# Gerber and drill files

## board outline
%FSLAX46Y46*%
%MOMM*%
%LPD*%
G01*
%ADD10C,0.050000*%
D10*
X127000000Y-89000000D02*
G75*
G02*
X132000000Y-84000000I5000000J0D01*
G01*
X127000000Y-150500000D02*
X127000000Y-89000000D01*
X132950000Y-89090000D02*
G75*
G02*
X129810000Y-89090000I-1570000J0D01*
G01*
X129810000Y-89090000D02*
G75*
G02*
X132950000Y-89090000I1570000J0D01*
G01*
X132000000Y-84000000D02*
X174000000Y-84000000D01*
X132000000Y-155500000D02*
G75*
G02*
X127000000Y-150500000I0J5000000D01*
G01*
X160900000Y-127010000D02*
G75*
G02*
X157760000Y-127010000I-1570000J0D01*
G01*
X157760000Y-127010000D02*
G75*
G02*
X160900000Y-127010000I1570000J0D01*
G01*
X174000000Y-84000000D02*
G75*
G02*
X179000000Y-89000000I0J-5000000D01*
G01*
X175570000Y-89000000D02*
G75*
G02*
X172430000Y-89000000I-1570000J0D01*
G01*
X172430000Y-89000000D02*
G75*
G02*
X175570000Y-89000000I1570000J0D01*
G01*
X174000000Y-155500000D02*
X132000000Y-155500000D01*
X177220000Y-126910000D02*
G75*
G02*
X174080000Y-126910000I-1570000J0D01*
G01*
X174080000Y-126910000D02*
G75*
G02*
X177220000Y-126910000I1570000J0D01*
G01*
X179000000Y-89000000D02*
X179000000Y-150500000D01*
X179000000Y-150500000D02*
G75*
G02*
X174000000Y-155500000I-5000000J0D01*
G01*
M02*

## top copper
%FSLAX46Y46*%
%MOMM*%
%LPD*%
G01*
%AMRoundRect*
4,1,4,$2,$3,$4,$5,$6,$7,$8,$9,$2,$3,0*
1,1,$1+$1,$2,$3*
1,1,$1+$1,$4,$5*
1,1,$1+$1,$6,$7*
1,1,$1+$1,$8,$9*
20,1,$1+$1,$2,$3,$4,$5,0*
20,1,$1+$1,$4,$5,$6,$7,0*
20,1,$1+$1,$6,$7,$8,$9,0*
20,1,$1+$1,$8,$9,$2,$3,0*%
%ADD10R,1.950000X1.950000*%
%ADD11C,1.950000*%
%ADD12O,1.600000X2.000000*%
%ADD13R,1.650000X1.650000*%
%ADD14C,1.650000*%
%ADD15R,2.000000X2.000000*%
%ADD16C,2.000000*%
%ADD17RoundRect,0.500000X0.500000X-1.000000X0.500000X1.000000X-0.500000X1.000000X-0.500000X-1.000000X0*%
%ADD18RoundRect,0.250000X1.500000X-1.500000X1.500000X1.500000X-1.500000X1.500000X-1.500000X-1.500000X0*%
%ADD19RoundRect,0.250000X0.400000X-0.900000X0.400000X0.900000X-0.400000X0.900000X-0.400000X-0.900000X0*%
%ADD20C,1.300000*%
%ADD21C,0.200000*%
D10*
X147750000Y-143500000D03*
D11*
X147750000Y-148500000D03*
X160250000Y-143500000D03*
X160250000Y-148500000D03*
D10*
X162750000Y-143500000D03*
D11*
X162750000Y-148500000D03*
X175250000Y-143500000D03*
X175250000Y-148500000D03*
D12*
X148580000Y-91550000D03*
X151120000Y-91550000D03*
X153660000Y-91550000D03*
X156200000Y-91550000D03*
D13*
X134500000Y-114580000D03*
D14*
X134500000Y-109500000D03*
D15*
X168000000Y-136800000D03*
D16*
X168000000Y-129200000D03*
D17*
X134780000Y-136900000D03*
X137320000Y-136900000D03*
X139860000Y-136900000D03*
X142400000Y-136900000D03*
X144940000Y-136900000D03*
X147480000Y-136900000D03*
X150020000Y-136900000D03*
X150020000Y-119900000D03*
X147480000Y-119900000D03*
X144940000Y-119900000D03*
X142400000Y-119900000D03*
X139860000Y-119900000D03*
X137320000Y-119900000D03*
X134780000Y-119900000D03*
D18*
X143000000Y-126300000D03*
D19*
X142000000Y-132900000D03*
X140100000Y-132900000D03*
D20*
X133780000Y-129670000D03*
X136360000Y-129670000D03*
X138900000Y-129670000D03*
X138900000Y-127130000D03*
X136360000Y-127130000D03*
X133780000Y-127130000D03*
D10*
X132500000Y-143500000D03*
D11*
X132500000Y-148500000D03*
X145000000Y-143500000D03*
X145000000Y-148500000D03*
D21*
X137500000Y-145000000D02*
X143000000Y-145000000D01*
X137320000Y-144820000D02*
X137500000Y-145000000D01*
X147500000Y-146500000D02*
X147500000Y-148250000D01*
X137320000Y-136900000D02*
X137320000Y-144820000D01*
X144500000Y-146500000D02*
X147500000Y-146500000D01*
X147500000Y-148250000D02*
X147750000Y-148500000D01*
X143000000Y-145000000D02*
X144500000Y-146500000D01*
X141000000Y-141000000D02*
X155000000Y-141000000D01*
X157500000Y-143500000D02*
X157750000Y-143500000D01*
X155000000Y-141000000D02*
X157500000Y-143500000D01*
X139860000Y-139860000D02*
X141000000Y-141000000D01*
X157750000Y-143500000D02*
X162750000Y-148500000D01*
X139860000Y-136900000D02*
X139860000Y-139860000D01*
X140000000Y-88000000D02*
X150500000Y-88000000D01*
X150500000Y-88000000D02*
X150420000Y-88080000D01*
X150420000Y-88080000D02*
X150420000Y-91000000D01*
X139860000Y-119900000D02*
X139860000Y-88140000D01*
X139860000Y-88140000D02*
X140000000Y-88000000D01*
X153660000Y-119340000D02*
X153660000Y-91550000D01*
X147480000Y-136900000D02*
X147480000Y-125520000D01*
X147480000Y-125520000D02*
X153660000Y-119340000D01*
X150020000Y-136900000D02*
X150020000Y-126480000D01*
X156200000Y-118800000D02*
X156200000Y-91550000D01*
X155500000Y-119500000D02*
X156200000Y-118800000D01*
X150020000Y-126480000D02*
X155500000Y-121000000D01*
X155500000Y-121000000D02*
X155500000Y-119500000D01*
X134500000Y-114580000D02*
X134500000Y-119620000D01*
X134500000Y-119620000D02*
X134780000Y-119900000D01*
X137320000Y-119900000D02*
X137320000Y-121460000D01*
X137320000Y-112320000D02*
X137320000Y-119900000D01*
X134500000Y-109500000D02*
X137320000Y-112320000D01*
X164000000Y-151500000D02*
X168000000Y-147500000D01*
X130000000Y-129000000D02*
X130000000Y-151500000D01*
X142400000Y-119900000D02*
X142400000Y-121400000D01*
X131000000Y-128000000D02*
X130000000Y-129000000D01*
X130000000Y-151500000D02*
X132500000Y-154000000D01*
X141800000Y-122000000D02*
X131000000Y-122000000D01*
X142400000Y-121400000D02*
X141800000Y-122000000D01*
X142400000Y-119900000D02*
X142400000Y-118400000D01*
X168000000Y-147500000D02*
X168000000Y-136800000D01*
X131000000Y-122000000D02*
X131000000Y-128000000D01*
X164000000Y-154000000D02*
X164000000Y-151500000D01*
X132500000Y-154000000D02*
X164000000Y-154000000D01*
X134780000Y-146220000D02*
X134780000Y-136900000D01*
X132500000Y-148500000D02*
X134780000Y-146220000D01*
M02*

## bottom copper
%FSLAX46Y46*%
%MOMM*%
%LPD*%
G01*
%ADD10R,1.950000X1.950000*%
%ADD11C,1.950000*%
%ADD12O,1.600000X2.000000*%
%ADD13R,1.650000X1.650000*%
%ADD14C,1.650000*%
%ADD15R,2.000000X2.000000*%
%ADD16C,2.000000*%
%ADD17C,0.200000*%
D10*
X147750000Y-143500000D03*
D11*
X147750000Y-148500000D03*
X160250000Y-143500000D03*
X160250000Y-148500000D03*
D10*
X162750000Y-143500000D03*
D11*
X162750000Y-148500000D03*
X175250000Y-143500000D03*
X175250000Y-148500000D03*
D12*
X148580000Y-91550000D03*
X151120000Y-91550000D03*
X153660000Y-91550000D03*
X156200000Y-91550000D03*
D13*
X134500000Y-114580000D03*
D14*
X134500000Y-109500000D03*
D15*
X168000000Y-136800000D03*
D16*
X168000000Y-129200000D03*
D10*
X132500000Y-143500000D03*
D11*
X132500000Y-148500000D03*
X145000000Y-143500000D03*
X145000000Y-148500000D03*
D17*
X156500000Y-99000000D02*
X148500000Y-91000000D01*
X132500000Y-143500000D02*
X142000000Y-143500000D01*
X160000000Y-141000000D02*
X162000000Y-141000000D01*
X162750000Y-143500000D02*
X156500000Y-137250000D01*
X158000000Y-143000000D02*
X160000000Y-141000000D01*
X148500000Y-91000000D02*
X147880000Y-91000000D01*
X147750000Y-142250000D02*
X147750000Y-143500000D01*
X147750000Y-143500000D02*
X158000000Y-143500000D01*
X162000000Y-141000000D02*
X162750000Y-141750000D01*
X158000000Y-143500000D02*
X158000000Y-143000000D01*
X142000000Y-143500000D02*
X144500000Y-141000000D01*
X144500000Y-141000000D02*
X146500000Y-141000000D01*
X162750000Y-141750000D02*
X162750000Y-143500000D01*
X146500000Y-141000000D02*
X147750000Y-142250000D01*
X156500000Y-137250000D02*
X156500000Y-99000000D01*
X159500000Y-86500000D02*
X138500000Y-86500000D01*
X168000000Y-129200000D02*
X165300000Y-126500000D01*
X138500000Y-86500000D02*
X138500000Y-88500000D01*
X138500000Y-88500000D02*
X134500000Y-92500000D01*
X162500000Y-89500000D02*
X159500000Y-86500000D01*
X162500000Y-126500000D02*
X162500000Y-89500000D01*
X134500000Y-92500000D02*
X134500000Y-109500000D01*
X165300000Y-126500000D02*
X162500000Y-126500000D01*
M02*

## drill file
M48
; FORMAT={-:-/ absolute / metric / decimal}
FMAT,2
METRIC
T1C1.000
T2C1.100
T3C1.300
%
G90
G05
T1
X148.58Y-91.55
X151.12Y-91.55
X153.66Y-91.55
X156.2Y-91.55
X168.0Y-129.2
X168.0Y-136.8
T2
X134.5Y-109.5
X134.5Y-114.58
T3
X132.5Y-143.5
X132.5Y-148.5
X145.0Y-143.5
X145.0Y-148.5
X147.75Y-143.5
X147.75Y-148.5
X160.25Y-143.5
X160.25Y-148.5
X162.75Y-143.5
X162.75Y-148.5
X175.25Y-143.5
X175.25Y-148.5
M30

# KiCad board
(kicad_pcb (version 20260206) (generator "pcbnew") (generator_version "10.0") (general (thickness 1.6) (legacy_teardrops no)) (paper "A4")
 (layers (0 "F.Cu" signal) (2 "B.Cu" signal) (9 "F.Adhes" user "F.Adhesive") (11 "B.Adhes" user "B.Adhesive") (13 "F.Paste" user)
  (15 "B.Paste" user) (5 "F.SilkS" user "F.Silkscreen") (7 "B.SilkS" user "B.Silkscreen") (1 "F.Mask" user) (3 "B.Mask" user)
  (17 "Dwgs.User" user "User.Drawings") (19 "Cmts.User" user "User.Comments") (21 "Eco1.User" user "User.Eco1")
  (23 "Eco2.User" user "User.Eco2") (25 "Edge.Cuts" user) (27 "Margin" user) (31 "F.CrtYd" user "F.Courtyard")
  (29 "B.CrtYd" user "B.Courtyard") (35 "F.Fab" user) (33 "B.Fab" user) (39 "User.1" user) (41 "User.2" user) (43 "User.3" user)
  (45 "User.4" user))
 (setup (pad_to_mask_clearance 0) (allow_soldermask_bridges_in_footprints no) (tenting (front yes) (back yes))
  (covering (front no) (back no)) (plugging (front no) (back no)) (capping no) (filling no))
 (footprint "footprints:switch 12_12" (layer "F.Cu") (at 154 146)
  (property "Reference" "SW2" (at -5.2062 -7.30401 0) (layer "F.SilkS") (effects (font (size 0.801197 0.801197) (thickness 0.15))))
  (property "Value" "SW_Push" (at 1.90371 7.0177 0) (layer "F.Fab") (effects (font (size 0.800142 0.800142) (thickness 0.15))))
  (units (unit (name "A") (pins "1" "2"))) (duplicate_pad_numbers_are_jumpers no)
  (pad "1" thru_hole rect (at -6.25 -2.5) (size 1.95 1.95) (drill 1.3) (layers "*.Cu" "*.Mask") (remove_unused_layers no) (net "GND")
   (solder_mask_margin 0.102))
  (pad "2" thru_hole circle (at -6.25 2.5) (size 1.95 1.95) (drill 1.3) (layers "*.Cu" "*.Mask") (remove_unused_layers no)
   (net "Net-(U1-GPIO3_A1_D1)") (solder_mask_margin 0.102))
  (pad "3" thru_hole circle (at 6.25 -2.5) (size 1.95 1.95) (drill 1.3) (layers "*.Cu" "*.Mask") (remove_unused_layers no)
   (solder_mask_margin 0.102))
  (pad "4" thru_hole circle (at 6.25 2.5) (size 1.95 1.95) (drill 1.3) (layers "*.Cu" "*.Mask") (remove_unused_layers no)
   (solder_mask_margin 0.102)))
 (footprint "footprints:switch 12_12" (layer "F.Cu") (at 169 146)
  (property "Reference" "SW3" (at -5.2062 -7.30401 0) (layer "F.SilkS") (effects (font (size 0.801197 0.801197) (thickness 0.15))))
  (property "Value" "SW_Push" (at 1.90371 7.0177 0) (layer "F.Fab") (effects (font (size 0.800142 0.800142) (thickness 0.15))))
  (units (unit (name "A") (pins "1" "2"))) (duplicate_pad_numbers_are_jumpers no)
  (pad "1" thru_hole rect (at -6.25 -2.5) (size 1.95 1.95) (drill 1.3) (layers "*.Cu" "*.Mask") (remove_unused_layers no) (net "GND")
   (solder_mask_margin 0.102))
  (pad "2" thru_hole circle (at -6.25 2.5) (size 1.95 1.95) (drill 1.3) (layers "*.Cu" "*.Mask") (remove_unused_layers no)
   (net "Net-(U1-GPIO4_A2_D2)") (solder_mask_margin 0.102))
  (pad "3" thru_hole circle (at 6.25 -2.5) (size 1.95 1.95) (drill 1.3) (layers "*.Cu" "*.Mask") (remove_unused_layers no)
   (solder_mask_margin 0.102))
  (pad "4" thru_hole circle (at 6.25 2.5) (size 1.95 1.95) (drill 1.3) (layers "*.Cu" "*.Mask") (remove_unused_layers no)
   (solder_mask_margin 0.102)))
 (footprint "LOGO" (layer "F.Cu") (at 171 118)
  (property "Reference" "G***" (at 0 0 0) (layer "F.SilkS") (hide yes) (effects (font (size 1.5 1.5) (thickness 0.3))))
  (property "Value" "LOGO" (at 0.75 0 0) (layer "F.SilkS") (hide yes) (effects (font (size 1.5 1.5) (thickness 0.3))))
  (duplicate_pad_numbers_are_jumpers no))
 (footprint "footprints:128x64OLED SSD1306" (layer "F.Cu") (at 152.2 102.15)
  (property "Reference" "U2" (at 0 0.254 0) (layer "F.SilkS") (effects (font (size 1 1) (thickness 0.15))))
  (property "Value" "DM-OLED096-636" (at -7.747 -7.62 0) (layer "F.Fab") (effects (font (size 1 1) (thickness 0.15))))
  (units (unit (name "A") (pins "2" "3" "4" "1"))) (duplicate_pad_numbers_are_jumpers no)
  (pad "1" thru_hole oval (at -3.62 -10.6 90) (size 2 1.6) (drill 1) (layers "*.Cu" "*.Mask") (remove_unused_layers no) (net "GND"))
  (pad "2" thru_hole oval (at -1.08 -10.6 90) (size 2 1.6) (drill 1) (layers "*.Cu" "*.Mask") (remove_unused_layers no) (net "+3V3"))
  (pad "3" thru_hole oval (at 1.46 -10.6 90) (size 2 1.6) (drill 1) (layers "*.Cu" "*.Mask") (remove_unused_layers no)
   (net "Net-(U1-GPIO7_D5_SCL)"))
  (pad "4" thru_hole oval (at 4 -10.6 90) (size 2 1.6) (drill 1) (layers "*.Cu" "*.Mask") (remove_unused_layers no)
   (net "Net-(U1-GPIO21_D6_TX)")))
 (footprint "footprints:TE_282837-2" (layer "F.Cu") (at 134.5 112.04 90)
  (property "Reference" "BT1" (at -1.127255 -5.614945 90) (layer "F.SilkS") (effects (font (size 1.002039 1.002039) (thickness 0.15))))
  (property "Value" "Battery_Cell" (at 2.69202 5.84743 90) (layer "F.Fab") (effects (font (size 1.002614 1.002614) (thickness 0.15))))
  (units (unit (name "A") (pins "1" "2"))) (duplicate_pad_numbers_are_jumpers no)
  (pad "1" thru_hole rect (at -2.54 0 90) (size 1.65 1.65) (drill 1.1) (layers "*.Cu" "*.Mask") (remove_unused_layers no)
   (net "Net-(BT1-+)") (solder_mask_margin 0.102))
  (pad "2" thru_hole circle (at 2.54 0 90) (size 1.65 1.65) (drill 1.1) (layers "*.Cu" "*.Mask") (remove_unused_layers no)
   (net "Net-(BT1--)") (solder_mask_margin 0.102)))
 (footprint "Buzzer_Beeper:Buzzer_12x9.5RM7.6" (layer "F.Cu") (at 168 136.8 90)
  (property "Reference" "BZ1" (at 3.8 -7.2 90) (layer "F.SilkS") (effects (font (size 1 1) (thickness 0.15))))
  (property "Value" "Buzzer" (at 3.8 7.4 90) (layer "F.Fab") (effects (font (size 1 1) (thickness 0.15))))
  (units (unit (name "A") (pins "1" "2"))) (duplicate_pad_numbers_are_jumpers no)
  (pad "1" thru_hole rect (at 0 0 90) (size 2 2) (drill 1) (layers "*.Cu" "*.Mask") (remove_unused_layers no) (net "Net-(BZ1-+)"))
  (pad "2" thru_hole circle (at 7.6 0 90) (size 2 2) (drill 1) (layers "*.Cu" "*.Mask") (remove_unused_layers no) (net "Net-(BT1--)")))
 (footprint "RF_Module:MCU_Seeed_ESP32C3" (layer "F.Cu") (at 142.4 128.4 90)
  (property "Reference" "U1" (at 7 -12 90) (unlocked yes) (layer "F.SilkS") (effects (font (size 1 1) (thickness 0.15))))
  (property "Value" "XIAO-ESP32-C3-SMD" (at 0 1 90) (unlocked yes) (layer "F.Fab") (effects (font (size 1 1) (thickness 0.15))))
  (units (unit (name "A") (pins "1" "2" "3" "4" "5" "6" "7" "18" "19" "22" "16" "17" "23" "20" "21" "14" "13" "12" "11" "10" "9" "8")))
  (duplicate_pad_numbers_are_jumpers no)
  (pad "" smd roundrect (at 1.1 -0.4 90) (size 1.5 1.5) (layers "F.Paste") (roundrect_rratio 0.1666666667))
  (pad "" smd roundrect (at 1.1 1.6 90) (size 1.5 1.5) (layers "F.Paste") (roundrect_rratio 0.1666666667))
  (pad "" smd roundrect (at 3.1 -0.4 90) (size 1.5 1.5) (layers "F.Paste") (roundrect_rratio 0.1666666667))
  (pad "" smd roundrect (at 3.1 1.6 90) (size 1.5 1.5) (layers "F.Paste") (roundrect_rratio 0.1666666667))
  (pad "1" smd roundrect (at -8.5 -7.62 90) (size 3 2) (layers "F.Cu" "F.Mask" "F.Paste") (roundrect_rratio 0.25)
   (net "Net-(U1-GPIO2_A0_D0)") (thermal_bridge_angle 45))
  (pad "2" smd roundrect (at -8.5 -5.08 90) (size 3 2) (layers "F.Cu" "F.Mask" "F.Paste") (roundrect_rratio 0.25)
   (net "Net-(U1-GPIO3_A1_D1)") (thermal_bridge_angle 45))
  (pad "3" smd roundrect (at -8.5 -2.54 90) (size 3 2) (layers "F.Cu" "F.Mask" "F.Paste") (roundrect_rratio 0.25)
   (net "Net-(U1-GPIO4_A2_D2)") (thermal_bridge_angle 45))
  (pad "4" smd roundrect (at -8.5 0 90) (size 3 2) (layers "F.Cu" "F.Mask" "F.Paste") (roundrect_rratio 0.25)
   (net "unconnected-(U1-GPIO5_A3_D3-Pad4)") (thermal_bridge_angle 45))
  (pad "5" smd roundrect (at -8.5 2.54 90) (size 3 2) (layers "F.Cu" "F.Mask" "F.Paste") (roundrect_rratio 0.25)
   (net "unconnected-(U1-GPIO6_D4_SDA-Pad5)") (thermal_bridge_angle 45))
  (pad "6" smd roundrect (at -8.5 5.08 90) (size 3 2) (layers "F.Cu" "F.Mask" "F.Paste") (roundrect_rratio 0.25)
   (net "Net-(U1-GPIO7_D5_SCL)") (thermal_bridge_angle 45))
  (pad "7" smd roundrect (at -8.5 7.62 90) (size 3 2) (layers "F.Cu" "F.Mask" "F.Paste") (roundrect_rratio 0.25)
   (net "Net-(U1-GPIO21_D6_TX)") (thermal_bridge_angle 45))
  (pad "8" smd roundrect (at 8.5 7.62 90) (size 3 2) (layers "F.Cu" "F.Mask" "F.Paste") (roundrect_rratio 0.25)
   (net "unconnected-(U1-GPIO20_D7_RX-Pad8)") (thermal_bridge_angle 45))
  (pad "9" smd roundrect (at 8.5 5.08 90) (size 3 2) (layers "F.Cu" "F.Mask" "F.Paste") (roundrect_rratio 0.25)
   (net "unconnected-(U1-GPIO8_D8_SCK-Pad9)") (thermal_bridge_angle 45))
  (pad "10" smd roundrect (at 8.5 2.54 90) (size 3 2) (layers "F.Cu" "F.Mask" "F.Paste") (roundrect_rratio 0.25)
   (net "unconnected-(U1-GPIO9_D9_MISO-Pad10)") (thermal_bridge_angle 45))
  (pad "11" smd roundrect (at 8.5 0 90) (size 3 2) (layers "F.Cu" "F.Mask" "F.Paste") (roundrect_rratio 0.25) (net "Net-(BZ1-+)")
   (thermal_bridge_angle 45))
  (pad "12" smd roundrect (at 8.5 -2.54 90) (size 3 2) (layers "F.Cu" "F.Mask" "F.Paste") (roundrect_rratio 0.25) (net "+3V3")
   (thermal_bridge_angle 45))
  (pad "13" smd roundrect (at 8.5 -5.08 90) (size 3 2) (layers "F.Cu" "F.Mask" "F.Paste") (roundrect_rratio 0.25) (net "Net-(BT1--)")
   (thermal_bridge_angle 45))
  (pad "14" smd roundrect (at 8.5 -7.62 90) (size 3 2) (layers "F.Cu" "F.Mask" "F.Paste") (roundrect_rratio 0.25) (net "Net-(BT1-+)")
   (thermal_bridge_angle 45))
  (pad "15" smd roundrect (at 2.1 0.6 90) (size 3.5 3.5) (layers "F.Cu" "F.Mask") (roundrect_rratio 0.07142857143))
  (pad "16" smd roundrect (at -4.5 -0.4 90) (size 2.3 1.3) (layers "F.Cu" "F.Mask" "F.Paste") (roundrect_rratio 0.1923076923)
   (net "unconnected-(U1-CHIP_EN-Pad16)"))
  (pad "17" smd roundrect (at -4.5 -2.3 90) (size 2.3 1.3) (layers "F.Cu" "F.Mask" "F.Paste") (roundrect_rratio 0.1923076923)
   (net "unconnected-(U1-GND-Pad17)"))
  (pad "18" smd circle (at -1.27 -8.62 90) (size 1.3 1.3) (layers "F.Cu" "F.Mask" "F.Paste") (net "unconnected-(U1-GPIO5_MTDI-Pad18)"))
  (pad "19" smd circle (at -1.27 -6.04 90) (size 1.3 1.3) (layers "F.Cu" "F.Mask" "F.Paste") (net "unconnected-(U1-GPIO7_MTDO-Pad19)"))
  (pad "20" smd circle (at -1.27 -3.5 90) (size 1.3 1.3) (layers "F.Cu" "F.Mask" "F.Paste") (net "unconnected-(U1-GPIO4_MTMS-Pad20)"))
  (pad "21" smd circle (at 1.27 -3.5 90) (size 1.3 1.3) (layers "F.Cu" "F.Mask" "F.Paste") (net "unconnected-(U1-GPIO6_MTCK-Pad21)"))
  (pad "22" smd circle (at 1.27 -6.04 90) (size 1.3 1.3) (layers "F.Cu" "F.Mask" "F.Paste") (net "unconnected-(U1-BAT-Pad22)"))
  (pad "23" smd circle (at 1.27 -8.62 90) (size 1.3 1.3) (layers "F.Cu" "F.Mask" "F.Paste") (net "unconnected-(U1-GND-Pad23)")))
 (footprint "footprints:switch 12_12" (layer "F.Cu") (at 138.75 146)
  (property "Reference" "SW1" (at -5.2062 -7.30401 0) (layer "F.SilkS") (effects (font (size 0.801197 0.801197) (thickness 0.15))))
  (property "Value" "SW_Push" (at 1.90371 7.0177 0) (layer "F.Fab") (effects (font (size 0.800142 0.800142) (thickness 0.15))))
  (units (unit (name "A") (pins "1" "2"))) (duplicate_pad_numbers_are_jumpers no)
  (pad "1" thru_hole rect (at -6.25 -2.5) (size 1.95 1.95) (drill 1.3) (layers "*.Cu" "*.Mask") (remove_unused_layers no) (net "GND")
   (solder_mask_margin 0.102))
  (pad "2" thru_hole circle (at -6.25 2.5) (size 1.95 1.95) (drill 1.3) (layers "*.Cu" "*.Mask") (remove_unused_layers no)
   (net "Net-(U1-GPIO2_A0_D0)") (solder_mask_margin 0.102))
  (pad "3" thru_hole circle (at 6.25 -2.5) (size 1.95 1.95) (drill 1.3) (layers "*.Cu" "*.Mask") (remove_unused_layers no)
   (solder_mask_margin 0.102))
  (pad "4" thru_hole circle (at 6.25 2.5) (size 1.95 1.95) (drill 1.3) (layers "*.Cu" "*.Mask") (remove_unused_layers no)
   (solder_mask_margin 0.102)))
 (gr_arc (start 127 89) (mid 128.464466 85.464466) (end 132 84) (stroke (width 0.05) (type default)) (layer "Edge.Cuts"))
 (gr_line (start 127 150.5) (end 127 89) (stroke (width 0.05) (type default)) (layer "Edge.Cuts"))
 (gr_circle (center 131.38 89.09) (end 129.81 89.09) (stroke (width 0.05) (type default)) (fill no) (layer "Edge.Cuts"))
 (gr_line (start 132 84) (end 174 84) (stroke (width 0.05) (type default)) (layer "Edge.Cuts"))
 (gr_arc (start 132 155.5) (mid 128.464466 154.035534) (end 127 150.5) (stroke (width 0.05) (type default)) (layer "Edge.Cuts"))
 (gr_circle (center 159.33 127.01) (end 157.76 127.01) (stroke (width 0.05) (type default)) (fill no) (layer "Edge.Cuts"))
 (gr_arc (start 174 84) (mid 177.535534 85.464466) (end 179 89) (stroke (width 0.05) (type default)) (layer "Edge.Cuts"))
 (gr_circle (center 174 89) (end 172.43 89) (stroke (width 0.05) (type default)) (fill no) (layer "Edge.Cuts"))
 (gr_line (start 174 155.5) (end 132 155.5) (stroke (width 0.05) (type default)) (layer "Edge.Cuts"))
 (gr_circle (center 175.65 126.91) (end 174.08 126.91) (stroke (width 0.05) (type default)) (fill no) (layer "Edge.Cuts"))
 (gr_line (start 179 89) (end 179 150.5) (stroke (width 0.05) (type default)) (layer "Edge.Cuts"))
 (gr_arc (start 179 150.5) (mid 177.535534 154.035534) (end 174 155.5) (stroke (width 0.05) (type default)) (layer "Edge.Cuts"))
 (segment (start 156.5 99) (end 148.5 91) (width 0.2) (layer "B.Cu") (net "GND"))
 (segment (start 132.5 143.5) (end 142 143.5) (width 0.2) (layer "B.Cu") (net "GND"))
 (segment (start 160 141) (end 162 141) (width 0.2) (layer "B.Cu") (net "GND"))
 (segment (start 162.75 143.5) (end 156.5 137.25) (width 0.2) (layer "B.Cu") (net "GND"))
 (segment (start 158 143) (end 160 141) (width 0.2) (layer "B.Cu") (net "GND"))
 (segment (start 148.5 91) (end 147.88 91) (width 0.2) (layer "B.Cu") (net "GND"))
 (segment (start 147.75 142.25) (end 147.75 143.5) (width 0.2) (layer "B.Cu") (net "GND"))
 (segment (start 147.75 143.5) (end 158 143.5) (width 0.2) (layer "B.Cu") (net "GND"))
 (segment (start 162 141) (end 162.75 141.75) (width 0.2) (layer "B.Cu") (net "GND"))
 (segment (start 158 143.5) (end 158 143) (width 0.2) (layer "B.Cu") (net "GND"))
 (segment (start 142 143.5) (end 144.5 141) (width 0.2) (layer "B.Cu") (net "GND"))
 (segment (start 144.5 141) (end 146.5 141) (width 0.2) (layer "B.Cu") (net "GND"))
 (segment (start 162.75 141.75) (end 162.75 143.5) (width 0.2) (layer "B.Cu") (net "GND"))
 (segment (start 146.5 141) (end 147.75 142.25) (width 0.2) (layer "B.Cu") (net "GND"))
 (segment (start 156.5 137.25) (end 156.5 99) (width 0.2) (layer "B.Cu") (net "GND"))
 (segment (start 137.5 145) (end 143 145) (width 0.2) (layer "F.Cu") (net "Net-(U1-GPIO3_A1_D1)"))
 (segment (start 137.32 144.82) (end 137.5 145) (width 0.2) (layer "F.Cu") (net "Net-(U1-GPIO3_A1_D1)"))
 (segment (start 147.5 146.5) (end 147.5 148.25) (width 0.2) (layer "F.Cu") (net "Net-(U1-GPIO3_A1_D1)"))
 (segment (start 137.32 136.9) (end 137.32 144.82) (width 0.2) (layer "F.Cu") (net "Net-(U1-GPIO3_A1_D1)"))
 (segment (start 144.5 146.5) (end 147.5 146.5) (width 0.2) (layer "F.Cu") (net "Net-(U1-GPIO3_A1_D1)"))
 (segment (start 147.5 148.25) (end 147.75 148.5) (width 0.2) (layer "F.Cu") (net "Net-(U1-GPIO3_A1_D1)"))
 (segment (start 143 145) (end 144.5 146.5) (width 0.2) (layer "F.Cu") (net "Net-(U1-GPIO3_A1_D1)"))
 (segment (start 141 141) (end 155 141) (width 0.2) (layer "F.Cu") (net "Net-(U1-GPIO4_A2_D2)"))
 (segment (start 157.5 143.5) (end 157.75 143.5) (width 0.2) (layer "F.Cu") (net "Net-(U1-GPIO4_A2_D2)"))
 (segment (start 155 141) (end 157.5 143.5) (width 0.2) (layer "F.Cu") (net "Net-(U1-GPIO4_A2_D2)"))
 (segment (start 139.86 139.86) (end 141 141) (width 0.2) (layer "F.Cu") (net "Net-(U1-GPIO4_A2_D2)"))
 (segment (start 157.75 143.5) (end 162.75 148.5) (width 0.2) (layer "F.Cu") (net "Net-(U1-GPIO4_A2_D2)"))
 (segment (start 139.86 136.9) (end 139.86 139.86) (width 0.2) (layer "F.Cu") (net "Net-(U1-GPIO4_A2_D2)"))
 (segment (start 140 88) (end 150.5 88) (width 0.2) (layer "F.Cu") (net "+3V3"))
 (segment (start 150.5 88) (end 150.42 88.08) (width 0.2) (layer "F.Cu") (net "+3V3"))
 (segment (start 150.42 88.08) (end 150.42 91) (width 0.2) (layer "F.Cu") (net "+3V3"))
 (segment (start 139.86 119.9) (end 139.86 88.14) (width 0.2) (layer "F.Cu") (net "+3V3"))
 (segment (start 139.86 88.14) (end 140 88) (width 0.2) (layer "F.Cu") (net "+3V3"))
 (segment (start 153.66 119.34) (end 153.66 91.55) (width 0.2) (layer "F.Cu") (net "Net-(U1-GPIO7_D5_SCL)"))
 (segment (start 147.48 136.9) (end 147.48 125.52) (width 0.2) (layer "F.Cu") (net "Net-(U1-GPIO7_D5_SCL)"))
 (segment (start 147.48 125.52) (end 153.66 119.34) (width 0.2) (layer "F.Cu") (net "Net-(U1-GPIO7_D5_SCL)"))
 (segment (start 150.02 136.9) (end 150.02 126.48) (width 0.2) (layer "F.Cu") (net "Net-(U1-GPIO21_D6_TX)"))
 (segment (start 156.2 118.8) (end 156.2 91.55) (width 0.2) (layer "F.Cu") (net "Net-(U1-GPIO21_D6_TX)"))
 (segment (start 155.5 119.5) (end 156.2 118.8) (width 0.2) (layer "F.Cu") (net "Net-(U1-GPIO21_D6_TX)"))
 (segment (start 150.02 126.48) (end 155.5 121) (width 0.2) (layer "F.Cu") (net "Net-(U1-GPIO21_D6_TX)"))
 (segment (start 155.5 121) (end 155.5 119.5) (width 0.2) (layer "F.Cu") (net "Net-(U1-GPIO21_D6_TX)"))
 (segment (start 134.5 114.58) (end 134.5 119.62) (width 0.2) (layer "F.Cu") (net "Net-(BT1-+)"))
 (segment (start 134.5 119.62) (end 134.78 119.9) (width 0.2) (layer "F.Cu") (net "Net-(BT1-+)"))
 (segment (start 137.32 119.9) (end 137.32 121.46) (width 0.2) (layer "F.Cu") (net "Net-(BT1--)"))
 (segment (start 137.32 112.32) (end 137.32 119.9) (width 0.2) (layer "F.Cu") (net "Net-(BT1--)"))
 (segment (start 134.5 109.5) (end 137.32 112.32) (width 0.2) (layer "F.Cu") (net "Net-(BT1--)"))
 (segment (start 159.5 86.5) (end 138.5 86.5) (width 0.2) (layer "B.Cu") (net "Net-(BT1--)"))
 (segment (start 168 129.2) (end 165.3 126.5) (width 0.2) (layer "B.Cu") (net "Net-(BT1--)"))
 (segment (start 138.5 86.5) (end 138.5 88.5) (width 0.2) (layer "B.Cu") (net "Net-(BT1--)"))
 (segment (start 138.5 88.5) (end 134.5 92.5) (width 0.2) (layer "B.Cu") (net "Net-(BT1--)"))
 (segment (start 162.5 89.5) (end 159.5 86.5) (width 0.2) (layer "B.Cu") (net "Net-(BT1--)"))
 (segment (start 162.5 126.5) (end 162.5 89.5) (width 0.2) (layer "B.Cu") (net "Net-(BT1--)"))
 (segment (start 134.5 92.5) (end 134.5 109.5) (width 0.2) (layer "B.Cu") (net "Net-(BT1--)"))
 (segment (start 165.3 126.5) (end 162.5 126.5) (width 0.2) (layer "B.Cu") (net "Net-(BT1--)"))
 (segment (start 164 151.5) (end 168 147.5) (width 0.2) (layer "F.Cu") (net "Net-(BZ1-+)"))
 (segment (start 130 129) (end 130 151.5) (width 0.2) (layer "F.Cu") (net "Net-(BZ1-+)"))
 (segment (start 142.4 119.9) (end 142.4 121.4) (width 0.2) (layer "F.Cu") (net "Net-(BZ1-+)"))
 (segment (start 131 128) (end 130 129) (width 0.2) (layer "F.Cu") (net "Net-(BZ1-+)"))
 (segment (start 130 151.5) (end 132.5 154) (width 0.2) (layer "F.Cu") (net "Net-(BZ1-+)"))
 (segment (start 141.8 122) (end 131 122) (width 0.2) (layer "F.Cu") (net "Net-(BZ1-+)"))
 (segment (start 142.4 121.4) (end 141.8 122) (width 0.2) (layer "F.Cu") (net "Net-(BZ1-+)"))
 (segment (start 142.4 119.9) (end 142.4 118.4) (width 0.2) (layer "F.Cu") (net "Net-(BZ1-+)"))
 (segment (start 168 147.5) (end 168 136.8) (width 0.2) (layer "F.Cu") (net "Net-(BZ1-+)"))
 (segment (start 131 122) (end 131 128) (width 0.2) (layer "F.Cu") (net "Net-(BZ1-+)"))
 (segment (start 164 154) (end 164 151.5) (width 0.2) (layer "F.Cu") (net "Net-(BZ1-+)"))
 (segment (start 132.5 154) (end 164 154) (width 0.2) (layer "F.Cu") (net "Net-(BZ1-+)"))
 (segment (start 134.78 146.22) (end 134.78 136.9) (width 0.2) (layer "F.Cu") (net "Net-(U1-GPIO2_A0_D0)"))
 (segment (start 132.5 148.5) (end 134.78 146.22) (width 0.2) (layer "F.Cu") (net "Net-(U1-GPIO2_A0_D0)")))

